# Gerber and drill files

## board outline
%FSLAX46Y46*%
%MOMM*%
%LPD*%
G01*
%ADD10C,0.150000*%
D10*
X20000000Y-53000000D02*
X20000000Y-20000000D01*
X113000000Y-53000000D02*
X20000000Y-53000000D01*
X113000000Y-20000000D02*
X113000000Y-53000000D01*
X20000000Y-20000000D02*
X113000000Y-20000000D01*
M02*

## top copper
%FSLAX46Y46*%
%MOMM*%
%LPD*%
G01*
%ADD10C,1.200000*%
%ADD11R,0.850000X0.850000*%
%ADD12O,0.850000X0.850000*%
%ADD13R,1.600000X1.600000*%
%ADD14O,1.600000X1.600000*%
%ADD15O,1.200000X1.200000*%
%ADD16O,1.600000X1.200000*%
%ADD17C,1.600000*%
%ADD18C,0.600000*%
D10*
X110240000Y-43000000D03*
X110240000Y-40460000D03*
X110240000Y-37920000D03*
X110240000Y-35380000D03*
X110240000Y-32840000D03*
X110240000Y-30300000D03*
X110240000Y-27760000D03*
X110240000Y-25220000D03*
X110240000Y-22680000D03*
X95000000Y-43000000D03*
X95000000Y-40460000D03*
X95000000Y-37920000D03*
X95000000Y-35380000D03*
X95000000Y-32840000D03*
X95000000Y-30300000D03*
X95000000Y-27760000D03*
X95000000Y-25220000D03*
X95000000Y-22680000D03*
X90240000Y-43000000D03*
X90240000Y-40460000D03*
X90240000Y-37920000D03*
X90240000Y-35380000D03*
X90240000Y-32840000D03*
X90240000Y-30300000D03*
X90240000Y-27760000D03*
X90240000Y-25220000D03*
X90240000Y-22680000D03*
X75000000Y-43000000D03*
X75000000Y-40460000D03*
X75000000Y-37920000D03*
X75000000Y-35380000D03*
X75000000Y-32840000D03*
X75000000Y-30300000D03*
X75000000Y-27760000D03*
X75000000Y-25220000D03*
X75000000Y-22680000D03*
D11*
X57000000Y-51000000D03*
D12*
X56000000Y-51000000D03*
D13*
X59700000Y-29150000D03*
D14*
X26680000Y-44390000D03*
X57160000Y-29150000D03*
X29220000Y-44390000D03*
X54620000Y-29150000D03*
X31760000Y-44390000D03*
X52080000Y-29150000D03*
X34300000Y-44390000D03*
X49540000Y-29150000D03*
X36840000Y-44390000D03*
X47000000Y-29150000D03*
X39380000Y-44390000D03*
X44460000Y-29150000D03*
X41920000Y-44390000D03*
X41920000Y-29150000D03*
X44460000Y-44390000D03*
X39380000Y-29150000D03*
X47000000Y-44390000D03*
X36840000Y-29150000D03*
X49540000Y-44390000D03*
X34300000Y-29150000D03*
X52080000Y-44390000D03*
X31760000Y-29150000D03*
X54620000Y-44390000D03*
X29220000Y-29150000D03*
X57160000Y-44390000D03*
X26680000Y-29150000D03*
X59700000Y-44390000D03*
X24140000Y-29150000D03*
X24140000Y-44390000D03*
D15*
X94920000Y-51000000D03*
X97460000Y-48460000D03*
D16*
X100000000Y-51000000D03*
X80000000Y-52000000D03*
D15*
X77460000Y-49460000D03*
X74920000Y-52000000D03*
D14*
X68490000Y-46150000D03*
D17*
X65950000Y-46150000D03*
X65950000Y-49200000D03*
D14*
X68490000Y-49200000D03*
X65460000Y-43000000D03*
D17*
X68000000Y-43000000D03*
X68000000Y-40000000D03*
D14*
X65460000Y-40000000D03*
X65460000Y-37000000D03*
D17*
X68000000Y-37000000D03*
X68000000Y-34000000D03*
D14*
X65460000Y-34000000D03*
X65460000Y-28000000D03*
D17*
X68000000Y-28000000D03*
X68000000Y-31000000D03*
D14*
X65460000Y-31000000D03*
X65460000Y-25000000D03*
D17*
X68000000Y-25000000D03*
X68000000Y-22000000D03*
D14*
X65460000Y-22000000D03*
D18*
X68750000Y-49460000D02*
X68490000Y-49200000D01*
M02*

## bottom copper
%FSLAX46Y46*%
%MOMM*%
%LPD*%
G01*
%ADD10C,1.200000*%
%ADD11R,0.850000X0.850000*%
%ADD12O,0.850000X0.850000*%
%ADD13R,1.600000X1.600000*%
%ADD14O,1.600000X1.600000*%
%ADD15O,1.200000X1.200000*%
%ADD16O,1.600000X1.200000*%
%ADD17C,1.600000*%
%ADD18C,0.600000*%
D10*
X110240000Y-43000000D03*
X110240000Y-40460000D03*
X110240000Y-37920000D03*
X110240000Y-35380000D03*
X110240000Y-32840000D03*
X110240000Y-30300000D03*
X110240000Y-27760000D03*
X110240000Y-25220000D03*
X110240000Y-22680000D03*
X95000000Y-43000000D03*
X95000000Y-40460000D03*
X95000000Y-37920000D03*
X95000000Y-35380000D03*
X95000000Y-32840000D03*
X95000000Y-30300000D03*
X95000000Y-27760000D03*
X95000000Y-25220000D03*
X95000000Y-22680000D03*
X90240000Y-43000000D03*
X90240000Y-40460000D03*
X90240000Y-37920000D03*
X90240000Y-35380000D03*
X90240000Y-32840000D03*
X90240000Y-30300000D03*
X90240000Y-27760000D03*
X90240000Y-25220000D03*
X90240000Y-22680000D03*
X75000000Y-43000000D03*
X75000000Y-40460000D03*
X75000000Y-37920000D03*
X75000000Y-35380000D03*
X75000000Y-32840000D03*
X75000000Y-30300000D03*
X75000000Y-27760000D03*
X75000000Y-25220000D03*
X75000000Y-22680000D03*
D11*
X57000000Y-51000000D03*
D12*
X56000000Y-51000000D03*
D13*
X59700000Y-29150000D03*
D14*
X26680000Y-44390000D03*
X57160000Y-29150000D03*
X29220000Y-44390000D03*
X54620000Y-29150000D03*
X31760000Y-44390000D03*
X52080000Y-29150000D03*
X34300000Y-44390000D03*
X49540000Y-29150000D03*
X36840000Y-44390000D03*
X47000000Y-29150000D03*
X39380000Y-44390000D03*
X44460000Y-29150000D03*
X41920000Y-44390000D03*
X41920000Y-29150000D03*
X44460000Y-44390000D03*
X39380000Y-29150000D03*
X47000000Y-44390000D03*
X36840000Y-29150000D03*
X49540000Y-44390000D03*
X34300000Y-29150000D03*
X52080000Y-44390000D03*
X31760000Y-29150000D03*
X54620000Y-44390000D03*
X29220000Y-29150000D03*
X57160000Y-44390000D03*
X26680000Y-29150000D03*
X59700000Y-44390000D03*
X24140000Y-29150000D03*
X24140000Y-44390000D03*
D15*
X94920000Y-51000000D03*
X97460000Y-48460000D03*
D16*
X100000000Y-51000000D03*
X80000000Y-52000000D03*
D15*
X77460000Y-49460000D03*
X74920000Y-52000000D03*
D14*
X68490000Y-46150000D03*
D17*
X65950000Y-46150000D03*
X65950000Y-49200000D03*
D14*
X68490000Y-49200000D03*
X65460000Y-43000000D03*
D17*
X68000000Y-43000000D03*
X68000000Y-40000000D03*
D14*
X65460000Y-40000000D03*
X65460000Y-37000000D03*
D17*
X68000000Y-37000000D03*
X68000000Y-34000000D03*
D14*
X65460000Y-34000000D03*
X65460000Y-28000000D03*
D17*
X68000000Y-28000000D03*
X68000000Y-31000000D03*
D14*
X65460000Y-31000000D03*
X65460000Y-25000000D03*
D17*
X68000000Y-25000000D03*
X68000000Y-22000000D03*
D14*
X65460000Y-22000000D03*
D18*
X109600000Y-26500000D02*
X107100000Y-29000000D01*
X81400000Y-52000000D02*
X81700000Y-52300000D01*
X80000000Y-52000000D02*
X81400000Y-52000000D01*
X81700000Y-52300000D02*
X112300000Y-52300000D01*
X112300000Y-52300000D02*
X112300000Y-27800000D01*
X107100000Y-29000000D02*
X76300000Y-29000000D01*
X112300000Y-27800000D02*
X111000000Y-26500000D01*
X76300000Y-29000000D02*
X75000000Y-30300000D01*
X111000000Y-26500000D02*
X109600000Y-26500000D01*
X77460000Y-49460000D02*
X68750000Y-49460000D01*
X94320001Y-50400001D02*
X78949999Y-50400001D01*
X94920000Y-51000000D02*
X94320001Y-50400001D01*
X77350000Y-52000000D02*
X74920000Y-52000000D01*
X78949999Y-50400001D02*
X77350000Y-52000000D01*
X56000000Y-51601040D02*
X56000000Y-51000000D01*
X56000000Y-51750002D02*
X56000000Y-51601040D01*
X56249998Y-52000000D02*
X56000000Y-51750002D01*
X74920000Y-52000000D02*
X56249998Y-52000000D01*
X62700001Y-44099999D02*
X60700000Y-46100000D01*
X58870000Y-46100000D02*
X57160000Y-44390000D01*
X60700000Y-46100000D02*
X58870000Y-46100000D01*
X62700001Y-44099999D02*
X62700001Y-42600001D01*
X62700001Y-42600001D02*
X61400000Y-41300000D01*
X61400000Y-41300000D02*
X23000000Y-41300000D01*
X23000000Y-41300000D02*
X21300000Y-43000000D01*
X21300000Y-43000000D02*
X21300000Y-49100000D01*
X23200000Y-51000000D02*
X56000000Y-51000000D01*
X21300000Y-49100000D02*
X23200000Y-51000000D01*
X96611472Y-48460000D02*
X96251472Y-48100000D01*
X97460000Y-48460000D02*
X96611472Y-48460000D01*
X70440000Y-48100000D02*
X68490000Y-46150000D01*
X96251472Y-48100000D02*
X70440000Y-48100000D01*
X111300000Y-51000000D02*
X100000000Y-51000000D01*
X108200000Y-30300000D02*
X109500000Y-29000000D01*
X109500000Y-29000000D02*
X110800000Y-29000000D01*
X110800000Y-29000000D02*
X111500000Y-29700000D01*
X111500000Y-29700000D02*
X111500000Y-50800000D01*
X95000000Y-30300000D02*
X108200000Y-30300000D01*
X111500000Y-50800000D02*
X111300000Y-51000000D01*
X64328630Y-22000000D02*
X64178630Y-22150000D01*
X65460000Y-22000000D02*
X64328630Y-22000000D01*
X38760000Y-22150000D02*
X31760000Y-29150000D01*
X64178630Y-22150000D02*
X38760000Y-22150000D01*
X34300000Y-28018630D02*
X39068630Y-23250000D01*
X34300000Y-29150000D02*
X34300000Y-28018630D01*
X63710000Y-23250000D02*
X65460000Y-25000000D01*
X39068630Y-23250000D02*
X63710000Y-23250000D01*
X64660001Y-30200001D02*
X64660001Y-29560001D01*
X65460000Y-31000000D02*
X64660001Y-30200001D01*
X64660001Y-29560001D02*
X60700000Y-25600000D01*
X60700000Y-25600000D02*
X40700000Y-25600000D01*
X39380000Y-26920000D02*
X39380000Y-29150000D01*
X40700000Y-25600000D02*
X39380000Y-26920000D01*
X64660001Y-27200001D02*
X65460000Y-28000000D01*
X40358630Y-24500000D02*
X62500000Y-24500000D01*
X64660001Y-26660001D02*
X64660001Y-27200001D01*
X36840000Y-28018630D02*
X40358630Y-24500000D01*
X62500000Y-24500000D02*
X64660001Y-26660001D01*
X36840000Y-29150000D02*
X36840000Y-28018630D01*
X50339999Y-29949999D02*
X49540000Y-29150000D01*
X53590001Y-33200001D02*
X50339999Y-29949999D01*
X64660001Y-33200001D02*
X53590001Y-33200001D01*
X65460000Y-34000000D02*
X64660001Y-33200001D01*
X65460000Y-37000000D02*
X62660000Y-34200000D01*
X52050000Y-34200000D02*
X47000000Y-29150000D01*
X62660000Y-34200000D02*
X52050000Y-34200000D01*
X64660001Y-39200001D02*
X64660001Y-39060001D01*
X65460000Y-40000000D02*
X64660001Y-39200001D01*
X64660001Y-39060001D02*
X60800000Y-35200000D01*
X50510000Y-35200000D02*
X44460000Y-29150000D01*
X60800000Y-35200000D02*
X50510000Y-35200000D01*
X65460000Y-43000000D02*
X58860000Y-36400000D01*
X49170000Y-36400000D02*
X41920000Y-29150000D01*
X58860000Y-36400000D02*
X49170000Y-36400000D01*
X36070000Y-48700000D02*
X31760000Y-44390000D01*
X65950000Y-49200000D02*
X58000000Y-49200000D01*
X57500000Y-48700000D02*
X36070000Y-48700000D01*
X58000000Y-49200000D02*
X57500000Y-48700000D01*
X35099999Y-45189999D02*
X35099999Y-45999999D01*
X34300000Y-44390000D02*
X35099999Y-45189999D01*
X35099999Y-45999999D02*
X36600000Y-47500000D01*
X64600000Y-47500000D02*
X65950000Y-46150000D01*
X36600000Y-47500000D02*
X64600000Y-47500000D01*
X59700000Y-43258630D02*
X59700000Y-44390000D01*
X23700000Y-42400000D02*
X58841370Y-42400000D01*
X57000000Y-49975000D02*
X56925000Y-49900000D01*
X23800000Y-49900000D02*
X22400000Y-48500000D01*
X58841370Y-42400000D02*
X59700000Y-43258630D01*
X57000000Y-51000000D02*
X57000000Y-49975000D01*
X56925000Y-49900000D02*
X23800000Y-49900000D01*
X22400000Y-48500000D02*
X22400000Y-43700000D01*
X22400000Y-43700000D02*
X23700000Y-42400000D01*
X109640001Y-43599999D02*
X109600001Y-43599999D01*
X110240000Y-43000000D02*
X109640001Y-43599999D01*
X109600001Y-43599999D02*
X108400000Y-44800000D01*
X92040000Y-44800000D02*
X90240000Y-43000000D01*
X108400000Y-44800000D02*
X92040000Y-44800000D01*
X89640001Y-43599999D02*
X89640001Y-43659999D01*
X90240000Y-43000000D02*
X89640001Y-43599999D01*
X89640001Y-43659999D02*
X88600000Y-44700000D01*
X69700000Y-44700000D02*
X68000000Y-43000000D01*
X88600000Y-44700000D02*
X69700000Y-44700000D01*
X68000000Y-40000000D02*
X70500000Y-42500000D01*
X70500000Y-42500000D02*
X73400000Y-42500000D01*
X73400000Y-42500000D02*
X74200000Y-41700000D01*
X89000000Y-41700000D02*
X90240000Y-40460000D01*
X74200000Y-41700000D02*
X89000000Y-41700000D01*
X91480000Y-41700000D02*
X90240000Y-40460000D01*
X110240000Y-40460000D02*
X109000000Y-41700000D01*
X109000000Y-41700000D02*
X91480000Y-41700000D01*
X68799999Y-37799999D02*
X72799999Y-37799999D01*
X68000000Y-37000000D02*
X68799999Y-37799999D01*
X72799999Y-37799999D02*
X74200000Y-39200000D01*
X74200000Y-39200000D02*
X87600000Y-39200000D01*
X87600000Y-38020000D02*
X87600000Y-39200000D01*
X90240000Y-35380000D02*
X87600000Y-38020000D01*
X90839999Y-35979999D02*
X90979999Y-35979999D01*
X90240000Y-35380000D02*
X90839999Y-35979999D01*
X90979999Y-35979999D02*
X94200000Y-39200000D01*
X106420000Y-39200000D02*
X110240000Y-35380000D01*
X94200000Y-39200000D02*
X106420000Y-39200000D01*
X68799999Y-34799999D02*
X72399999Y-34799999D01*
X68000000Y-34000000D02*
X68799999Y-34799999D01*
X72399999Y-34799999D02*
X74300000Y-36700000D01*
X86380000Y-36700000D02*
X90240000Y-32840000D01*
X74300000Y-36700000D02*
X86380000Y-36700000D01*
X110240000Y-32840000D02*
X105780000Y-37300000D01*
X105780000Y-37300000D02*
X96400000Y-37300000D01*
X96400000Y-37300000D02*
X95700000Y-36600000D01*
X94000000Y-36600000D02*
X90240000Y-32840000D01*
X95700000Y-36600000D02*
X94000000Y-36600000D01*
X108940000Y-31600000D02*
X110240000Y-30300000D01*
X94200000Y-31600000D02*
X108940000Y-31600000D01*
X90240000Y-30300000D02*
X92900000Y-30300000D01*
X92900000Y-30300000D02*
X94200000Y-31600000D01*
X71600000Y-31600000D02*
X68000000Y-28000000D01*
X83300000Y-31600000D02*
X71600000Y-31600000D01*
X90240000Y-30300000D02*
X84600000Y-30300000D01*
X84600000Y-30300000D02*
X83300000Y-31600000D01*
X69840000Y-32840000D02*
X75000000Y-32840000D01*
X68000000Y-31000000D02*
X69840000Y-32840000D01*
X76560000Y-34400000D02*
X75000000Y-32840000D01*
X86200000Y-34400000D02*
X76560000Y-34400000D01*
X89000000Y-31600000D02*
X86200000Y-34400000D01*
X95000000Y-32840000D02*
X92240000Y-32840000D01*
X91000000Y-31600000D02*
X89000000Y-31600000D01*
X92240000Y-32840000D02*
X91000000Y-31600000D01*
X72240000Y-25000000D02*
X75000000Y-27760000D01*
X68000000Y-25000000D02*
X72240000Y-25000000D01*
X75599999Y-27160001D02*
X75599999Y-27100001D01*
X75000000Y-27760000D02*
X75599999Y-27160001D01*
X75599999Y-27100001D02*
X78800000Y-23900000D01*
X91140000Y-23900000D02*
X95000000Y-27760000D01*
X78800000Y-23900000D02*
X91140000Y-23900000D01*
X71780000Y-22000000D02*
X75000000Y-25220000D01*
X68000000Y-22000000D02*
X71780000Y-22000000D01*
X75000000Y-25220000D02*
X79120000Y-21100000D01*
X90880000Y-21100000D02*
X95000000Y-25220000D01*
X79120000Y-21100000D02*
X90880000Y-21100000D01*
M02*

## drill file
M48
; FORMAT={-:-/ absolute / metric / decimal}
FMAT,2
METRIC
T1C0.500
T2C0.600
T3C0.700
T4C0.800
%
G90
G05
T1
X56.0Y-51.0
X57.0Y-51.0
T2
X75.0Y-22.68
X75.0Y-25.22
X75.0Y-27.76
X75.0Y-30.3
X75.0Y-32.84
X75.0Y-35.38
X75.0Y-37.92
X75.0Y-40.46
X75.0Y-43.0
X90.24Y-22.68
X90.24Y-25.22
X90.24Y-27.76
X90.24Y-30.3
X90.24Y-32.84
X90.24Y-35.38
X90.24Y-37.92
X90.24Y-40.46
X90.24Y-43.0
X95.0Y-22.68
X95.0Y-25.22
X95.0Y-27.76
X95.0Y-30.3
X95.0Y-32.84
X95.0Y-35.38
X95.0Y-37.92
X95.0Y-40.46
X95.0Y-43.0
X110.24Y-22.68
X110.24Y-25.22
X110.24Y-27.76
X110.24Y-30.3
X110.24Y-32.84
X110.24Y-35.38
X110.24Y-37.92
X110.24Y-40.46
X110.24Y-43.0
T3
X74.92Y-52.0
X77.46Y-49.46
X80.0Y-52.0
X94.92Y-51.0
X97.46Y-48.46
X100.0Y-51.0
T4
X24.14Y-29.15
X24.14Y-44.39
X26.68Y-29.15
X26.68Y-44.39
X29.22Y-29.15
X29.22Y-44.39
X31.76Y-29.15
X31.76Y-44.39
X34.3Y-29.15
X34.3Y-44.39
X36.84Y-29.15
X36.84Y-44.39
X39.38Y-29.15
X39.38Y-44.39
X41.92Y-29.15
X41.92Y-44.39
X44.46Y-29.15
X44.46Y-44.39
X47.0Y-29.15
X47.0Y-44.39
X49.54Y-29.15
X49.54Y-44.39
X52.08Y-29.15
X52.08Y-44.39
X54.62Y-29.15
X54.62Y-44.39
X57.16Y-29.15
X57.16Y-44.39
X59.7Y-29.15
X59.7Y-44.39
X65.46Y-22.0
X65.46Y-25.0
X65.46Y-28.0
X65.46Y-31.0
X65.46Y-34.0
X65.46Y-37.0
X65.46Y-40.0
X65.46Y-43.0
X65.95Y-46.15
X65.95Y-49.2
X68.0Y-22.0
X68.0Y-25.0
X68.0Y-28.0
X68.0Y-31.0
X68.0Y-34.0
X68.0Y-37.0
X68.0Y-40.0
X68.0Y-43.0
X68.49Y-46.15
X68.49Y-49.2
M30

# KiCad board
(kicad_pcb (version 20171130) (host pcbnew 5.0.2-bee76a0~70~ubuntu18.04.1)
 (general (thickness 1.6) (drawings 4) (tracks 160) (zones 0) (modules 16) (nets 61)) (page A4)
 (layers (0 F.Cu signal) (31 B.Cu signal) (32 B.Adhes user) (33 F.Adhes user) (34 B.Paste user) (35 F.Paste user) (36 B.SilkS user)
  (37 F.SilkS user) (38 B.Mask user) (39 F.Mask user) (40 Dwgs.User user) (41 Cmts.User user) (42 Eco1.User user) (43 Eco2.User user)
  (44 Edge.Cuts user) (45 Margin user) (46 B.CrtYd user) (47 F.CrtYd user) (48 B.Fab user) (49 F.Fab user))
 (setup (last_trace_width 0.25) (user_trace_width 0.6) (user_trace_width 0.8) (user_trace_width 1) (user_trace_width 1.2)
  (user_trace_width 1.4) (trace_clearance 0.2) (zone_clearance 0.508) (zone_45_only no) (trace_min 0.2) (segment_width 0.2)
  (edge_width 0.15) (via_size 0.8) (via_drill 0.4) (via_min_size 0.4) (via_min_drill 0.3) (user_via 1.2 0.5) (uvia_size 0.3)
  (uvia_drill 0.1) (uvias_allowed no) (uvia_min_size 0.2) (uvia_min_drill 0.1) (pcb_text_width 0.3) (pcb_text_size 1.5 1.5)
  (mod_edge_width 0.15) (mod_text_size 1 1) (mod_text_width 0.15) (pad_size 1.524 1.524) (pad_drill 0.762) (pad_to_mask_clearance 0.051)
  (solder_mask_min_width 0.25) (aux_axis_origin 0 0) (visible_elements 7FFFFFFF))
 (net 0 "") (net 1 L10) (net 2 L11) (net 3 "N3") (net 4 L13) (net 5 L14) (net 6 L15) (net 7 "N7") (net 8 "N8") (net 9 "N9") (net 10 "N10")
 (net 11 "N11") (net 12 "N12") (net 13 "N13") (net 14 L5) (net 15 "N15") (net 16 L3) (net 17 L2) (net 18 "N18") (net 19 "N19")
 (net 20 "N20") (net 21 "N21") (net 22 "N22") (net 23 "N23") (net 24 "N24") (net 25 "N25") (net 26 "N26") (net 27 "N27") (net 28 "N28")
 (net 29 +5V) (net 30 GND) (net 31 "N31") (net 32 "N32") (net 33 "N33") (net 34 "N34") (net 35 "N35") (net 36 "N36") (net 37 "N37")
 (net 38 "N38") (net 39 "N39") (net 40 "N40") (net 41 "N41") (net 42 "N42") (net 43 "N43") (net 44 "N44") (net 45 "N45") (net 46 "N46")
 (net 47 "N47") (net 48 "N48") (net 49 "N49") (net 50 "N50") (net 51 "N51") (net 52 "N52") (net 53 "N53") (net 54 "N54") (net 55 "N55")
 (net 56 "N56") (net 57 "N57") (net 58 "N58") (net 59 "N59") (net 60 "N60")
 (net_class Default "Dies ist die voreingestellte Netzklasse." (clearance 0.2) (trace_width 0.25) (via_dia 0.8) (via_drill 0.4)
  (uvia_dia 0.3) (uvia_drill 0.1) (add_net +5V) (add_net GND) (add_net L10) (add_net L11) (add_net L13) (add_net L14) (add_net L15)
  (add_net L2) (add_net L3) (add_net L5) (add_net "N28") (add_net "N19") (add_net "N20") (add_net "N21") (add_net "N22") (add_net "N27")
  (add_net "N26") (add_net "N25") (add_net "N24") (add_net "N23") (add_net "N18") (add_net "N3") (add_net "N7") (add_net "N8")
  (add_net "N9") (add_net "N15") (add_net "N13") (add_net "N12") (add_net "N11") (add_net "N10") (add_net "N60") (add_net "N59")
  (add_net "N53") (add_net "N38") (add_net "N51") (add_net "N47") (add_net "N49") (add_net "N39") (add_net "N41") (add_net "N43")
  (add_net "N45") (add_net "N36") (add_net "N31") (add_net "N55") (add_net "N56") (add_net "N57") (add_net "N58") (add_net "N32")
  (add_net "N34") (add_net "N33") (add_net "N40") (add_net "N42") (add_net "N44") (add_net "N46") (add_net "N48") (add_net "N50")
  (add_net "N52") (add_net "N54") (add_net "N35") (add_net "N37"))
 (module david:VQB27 (layer F.Cu) (at 95 43)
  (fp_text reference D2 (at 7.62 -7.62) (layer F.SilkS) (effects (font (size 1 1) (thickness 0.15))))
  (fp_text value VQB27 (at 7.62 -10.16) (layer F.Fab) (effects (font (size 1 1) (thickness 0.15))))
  (pad 10 thru_hole circle (at 15.24 0) (size 1.2 1.2) (drill 0.6) (layers *.Cu *.Mask) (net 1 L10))
  (pad 11 thru_hole circle (at 15.24 -2.54) (size 1.2 1.2) (drill 0.6) (layers *.Cu *.Mask) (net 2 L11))
  (pad 12 thru_hole circle (at 15.24 -5.08) (size 1.2 1.2) (drill 0.6) (layers *.Cu *.Mask) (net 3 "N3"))
  (pad 13 thru_hole circle (at 15.24 -7.62) (size 1.2 1.2) (drill 0.6) (layers *.Cu *.Mask) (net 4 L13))
  (pad 14 thru_hole circle (at 15.24 -10.16) (size 1.2 1.2) (drill 0.6) (layers *.Cu *.Mask) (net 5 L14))
  (pad 15 thru_hole circle (at 15.24 -12.7) (size 1.2 1.2) (drill 0.6) (layers *.Cu *.Mask) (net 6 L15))
  (pad 16 thru_hole circle (at 15.24 -15.24) (size 1.2 1.2) (drill 0.6) (layers *.Cu *.Mask) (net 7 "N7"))
  (pad 17 thru_hole circle (at 15.24 -17.78) (size 1.2 1.2) (drill 0.6) (layers *.Cu *.Mask) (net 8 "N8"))
  (pad 18 thru_hole circle (at 15.24 -20.32) (size 1.2 1.2) (drill 0.6) (layers *.Cu *.Mask) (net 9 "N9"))
  (pad 9 thru_hole circle (at 0 0) (size 1.2 1.2) (drill 0.6) (layers *.Cu *.Mask) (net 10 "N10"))
  (pad 8 thru_hole circle (at 0 -2.54) (size 1.2 1.2) (drill 0.6) (layers *.Cu *.Mask) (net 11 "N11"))
  (pad 7 thru_hole circle (at 0 -5.08) (size 1.2 1.2) (drill 0.6) (layers *.Cu *.Mask) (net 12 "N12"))
  (pad 6 thru_hole circle (at 0 -7.62) (size 1.2 1.2) (drill 0.6) (layers *.Cu *.Mask) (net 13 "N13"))
  (pad 5 thru_hole circle (at 0 -10.16) (size 1.2 1.2) (drill 0.6) (layers *.Cu *.Mask) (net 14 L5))
  (pad 4 thru_hole circle (at 0 -12.7) (size 1.2 1.2) (drill 0.6) (layers *.Cu *.Mask) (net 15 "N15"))
  (pad 3 thru_hole circle (at 0 -15.24) (size 1.2 1.2) (drill 0.6) (layers *.Cu *.Mask) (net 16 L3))
  (pad 2 thru_hole circle (at 0 -17.78) (size 1.2 1.2) (drill 0.6) (layers *.Cu *.Mask) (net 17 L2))
  (pad 1 thru_hole circle (at 0 -20.32) (size 1.2 1.2) (drill 0.6) (layers *.Cu *.Mask) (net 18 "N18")))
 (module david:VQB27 (layer F.Cu) (at 75 43)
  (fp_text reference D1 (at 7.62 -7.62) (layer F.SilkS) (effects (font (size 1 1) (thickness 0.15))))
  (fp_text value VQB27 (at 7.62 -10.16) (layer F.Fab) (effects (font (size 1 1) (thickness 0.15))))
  (pad 10 thru_hole circle (at 15.24 0) (size 1.2 1.2) (drill 0.6) (layers *.Cu *.Mask) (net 1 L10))
  (pad 11 thru_hole circle (at 15.24 -2.54) (size 1.2 1.2) (drill 0.6) (layers *.Cu *.Mask) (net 2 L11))
  (pad 12 thru_hole circle (at 15.24 -5.08) (size 1.2 1.2) (drill 0.6) (layers *.Cu *.Mask) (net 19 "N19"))
  (pad 13 thru_hole circle (at 15.24 -7.62) (size 1.2 1.2) (drill 0.6) (layers *.Cu *.Mask) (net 4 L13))
  (pad 14 thru_hole circle (at 15.24 -10.16) (size 1.2 1.2) (drill 0.6) (layers *.Cu *.Mask) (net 5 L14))
  (pad 15 thru_hole circle (at 15.24 -12.7) (size 1.2 1.2) (drill 0.6) (layers *.Cu *.Mask) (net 6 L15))
  (pad 16 thru_hole circle (at 15.24 -15.24) (size 1.2 1.2) (drill 0.6) (layers *.Cu *.Mask) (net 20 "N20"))
  (pad 17 thru_hole circle (at 15.24 -17.78) (size 1.2 1.2) (drill 0.6) (layers *.Cu *.Mask) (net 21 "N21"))
  (pad 18 thru_hole circle (at 15.24 -20.32) (size 1.2 1.2) (drill 0.6) (layers *.Cu *.Mask) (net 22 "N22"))
  (pad 9 thru_hole circle (at 0 0) (size 1.2 1.2) (drill 0.6) (layers *.Cu *.Mask) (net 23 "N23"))
  (pad 8 thru_hole circle (at 0 -2.54) (size 1.2 1.2) (drill 0.6) (layers *.Cu *.Mask) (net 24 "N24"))
  (pad 7 thru_hole circle (at 0 -5.08) (size 1.2 1.2) (drill 0.6) (layers *.Cu *.Mask) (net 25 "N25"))
  (pad 6 thru_hole circle (at 0 -7.62) (size 1.2 1.2) (drill 0.6) (layers *.Cu *.Mask) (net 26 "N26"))
  (pad 5 thru_hole circle (at 0 -10.16) (size 1.2 1.2) (drill 0.6) (layers *.Cu *.Mask) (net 14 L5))
  (pad 4 thru_hole circle (at 0 -12.7) (size 1.2 1.2) (drill 0.6) (layers *.Cu *.Mask) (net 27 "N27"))
  (pad 3 thru_hole circle (at 0 -15.24) (size 1.2 1.2) (drill 0.6) (layers *.Cu *.Mask) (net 16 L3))
  (pad 2 thru_hole circle (at 0 -17.78) (size 1.2 1.2) (drill 0.6) (layers *.Cu *.Mask) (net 17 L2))
  (pad 1 thru_hole circle (at 0 -20.32) (size 1.2 1.2) (drill 0.6) (layers *.Cu *.Mask) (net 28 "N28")))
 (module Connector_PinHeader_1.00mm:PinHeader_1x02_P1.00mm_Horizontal (layer F.Cu) (at 57 51 270)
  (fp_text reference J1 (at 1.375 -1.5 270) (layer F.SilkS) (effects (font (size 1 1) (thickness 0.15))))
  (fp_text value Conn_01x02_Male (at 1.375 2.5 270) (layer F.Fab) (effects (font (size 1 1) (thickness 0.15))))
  (pad 1 thru_hole rect (at 0 0 270) (size 0.85 0.85) (drill 0.5) (layers *.Cu *.Mask) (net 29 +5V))
  (pad 2 thru_hole oval (at 0 1 270) (size 0.85 0.85) (drill 0.5) (layers *.Cu *.Mask) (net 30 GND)))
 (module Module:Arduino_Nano (layer F.Cu) (at 59.7 29.15 270)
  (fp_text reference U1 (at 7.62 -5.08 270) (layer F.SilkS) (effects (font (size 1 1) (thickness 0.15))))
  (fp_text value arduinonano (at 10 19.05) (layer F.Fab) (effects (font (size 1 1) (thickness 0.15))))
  (pad 1 thru_hole rect (at 0 0 270) (size 1.6 1.6) (drill 0.8) (layers *.Cu *.Mask) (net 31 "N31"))
  (pad 17 thru_hole oval (at 15.24 33.02 270) (size 1.6 1.6) (drill 0.8) (layers *.Cu *.Mask) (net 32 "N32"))
  (pad 2 thru_hole oval (at 0 2.54 270) (size 1.6 1.6) (drill 0.8) (layers *.Cu *.Mask) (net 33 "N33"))
  (pad 18 thru_hole oval (at 15.24 30.48 270) (size 1.6 1.6) (drill 0.8) (layers *.Cu *.Mask) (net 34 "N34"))
  (pad 3 thru_hole oval (at 0 5.08 270) (size 1.6 1.6) (drill 0.8) (layers *.Cu *.Mask) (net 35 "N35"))
  (pad 19 thru_hole oval (at 15.24 27.94 270) (size 1.6 1.6) (drill 0.8) (layers *.Cu *.Mask) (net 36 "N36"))
  (pad 4 thru_hole oval (at 0 7.62 270) (size 1.6 1.6) (drill 0.8) (layers *.Cu *.Mask) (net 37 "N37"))
  (pad 20 thru_hole oval (at 15.24 25.4 270) (size 1.6 1.6) (drill 0.8) (layers *.Cu *.Mask) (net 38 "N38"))
  (pad 5 thru_hole oval (at 0 10.16 270) (size 1.6 1.6) (drill 0.8) (layers *.Cu *.Mask) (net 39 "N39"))
  (pad 21 thru_hole oval (at 15.24 22.86 270) (size 1.6 1.6) (drill 0.8) (layers *.Cu *.Mask) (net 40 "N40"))
  (pad 6 thru_hole oval (at 0 12.7 270) (size 1.6 1.6) (drill 0.8) (layers *.Cu *.Mask) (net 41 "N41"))
  (pad 22 thru_hole oval (at 15.24 20.32 270) (size 1.6 1.6) (drill 0.8) (layers *.Cu *.Mask) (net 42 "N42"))
  (pad 7 thru_hole oval (at 0 15.24 270) (size 1.6 1.6) (drill 0.8) (layers *.Cu *.Mask) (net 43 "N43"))
  (pad 23 thru_hole oval (at 15.24 17.78 270) (size 1.6 1.6) (drill 0.8) (layers *.Cu *.Mask) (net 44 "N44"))
  (pad 8 thru_hole oval (at 0 17.78 270) (size 1.6 1.6) (drill 0.8) (layers *.Cu *.Mask) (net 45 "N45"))
  (pad 24 thru_hole oval (at 15.24 15.24 270) (size 1.6 1.6) (drill 0.8) (layers *.Cu *.Mask) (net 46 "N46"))
  (pad 9 thru_hole oval (at 0 20.32 270) (size 1.6 1.6) (drill 0.8) (layers *.Cu *.Mask) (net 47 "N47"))
  (pad 25 thru_hole oval (at 15.24 12.7 270) (size 1.6 1.6) (drill 0.8) (layers *.Cu *.Mask) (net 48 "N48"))
  (pad 10 thru_hole oval (at 0 22.86 270) (size 1.6 1.6) (drill 0.8) (layers *.Cu *.Mask) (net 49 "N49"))
  (pad 26 thru_hole oval (at 15.24 10.16 270) (size 1.6 1.6) (drill 0.8) (layers *.Cu *.Mask) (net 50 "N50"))
  (pad 11 thru_hole oval (at 0 25.4 270) (size 1.6 1.6) (drill 0.8) (layers *.Cu *.Mask) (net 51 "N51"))
  (pad 27 thru_hole oval (at 15.24 7.62 270) (size 1.6 1.6) (drill 0.8) (layers *.Cu *.Mask) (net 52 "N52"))
  (pad 12 thru_hole oval (at 0 27.94 270) (size 1.6 1.6) (drill 0.8) (layers *.Cu *.Mask) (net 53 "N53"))
  (pad 28 thru_hole oval (at 15.24 5.08 270) (size 1.6 1.6) (drill 0.8) (layers *.Cu *.Mask) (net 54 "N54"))
  (pad 13 thru_hole oval (at 0 30.48 270) (size 1.6 1.6) (drill 0.8) (layers *.Cu *.Mask) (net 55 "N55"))
  (pad 29 thru_hole oval (at 15.24 2.54 270) (size 1.6 1.6) (drill 0.8) (layers *.Cu *.Mask) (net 30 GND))
  (pad 14 thru_hole oval (at 0 33.02 270) (size 1.6 1.6) (drill 0.8) (layers *.Cu *.Mask) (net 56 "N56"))
  (pad 30 thru_hole oval (at 15.24 0 270) (size 1.6 1.6) (drill 0.8) (layers *.Cu *.Mask) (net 29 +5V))
  (pad 15 thru_hole oval (at 0 35.56 270) (size 1.6 1.6) (drill 0.8) (layers *.Cu *.Mask) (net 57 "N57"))
  (pad 16 thru_hole oval (at 15.24 35.56 270) (size 1.6 1.6) (drill 0.8) (layers *.Cu *.Mask) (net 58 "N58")))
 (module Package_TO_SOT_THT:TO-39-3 (layer F.Cu) (at 100 51 180)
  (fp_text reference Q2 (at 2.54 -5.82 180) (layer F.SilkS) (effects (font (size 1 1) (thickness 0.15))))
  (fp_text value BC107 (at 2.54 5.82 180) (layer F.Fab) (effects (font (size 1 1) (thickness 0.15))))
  (pad 3 thru_hole oval (at 5.08 0 180) (size 1.2 1.2) (drill 0.7) (layers *.Cu *.Mask) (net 30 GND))
  (pad 2 thru_hole oval (at 2.54 2.54 180) (size 1.2 1.2) (drill 0.7) (layers *.Cu *.Mask) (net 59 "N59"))
  (pad 1 thru_hole oval (at 0 0 180) (size 1.6 1.2) (drill 0.7) (layers *.Cu *.Mask) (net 15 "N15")))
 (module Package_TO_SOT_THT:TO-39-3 (layer F.Cu) (at 80 52 180)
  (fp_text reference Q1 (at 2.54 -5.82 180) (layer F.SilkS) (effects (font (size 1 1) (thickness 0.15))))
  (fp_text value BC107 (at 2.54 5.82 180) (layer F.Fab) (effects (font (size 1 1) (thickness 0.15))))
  (pad 1 thru_hole oval (at 0 0 180) (size 1.6 1.2) (drill 0.7) (layers *.Cu *.Mask) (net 27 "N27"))
  (pad 2 thru_hole oval (at 2.54 2.54 180) (size 1.2 1.2) (drill 0.7) (layers *.Cu *.Mask) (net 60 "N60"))
  (pad 3 thru_hole oval (at 5.08 0 180) (size 1.2 1.2) (drill 0.7) (layers *.Cu *.Mask) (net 30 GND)))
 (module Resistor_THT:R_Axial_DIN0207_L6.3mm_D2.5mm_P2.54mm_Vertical (layer F.Cu) (at 65.95 46.15)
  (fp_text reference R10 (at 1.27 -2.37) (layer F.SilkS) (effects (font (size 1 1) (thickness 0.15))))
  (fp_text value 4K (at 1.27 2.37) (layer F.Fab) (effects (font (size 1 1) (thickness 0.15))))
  (pad 2 thru_hole oval (at 2.54 0) (size 1.6 1.6) (drill 0.8) (layers *.Cu *.Mask) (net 59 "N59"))
  (pad 1 thru_hole circle (at 0 0) (size 1.6 1.6) (drill 0.8) (layers *.Cu *.Mask) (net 38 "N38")))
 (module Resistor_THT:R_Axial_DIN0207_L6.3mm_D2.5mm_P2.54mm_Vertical (layer F.Cu) (at 65.95 49.2)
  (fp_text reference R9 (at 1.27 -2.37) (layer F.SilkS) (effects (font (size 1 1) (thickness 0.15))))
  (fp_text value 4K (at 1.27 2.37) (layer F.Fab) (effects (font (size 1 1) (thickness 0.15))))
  (pad 1 thru_hole circle (at 0 0) (size 1.6 1.6) (drill 0.8) (layers *.Cu *.Mask) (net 36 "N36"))
  (pad 2 thru_hole oval (at 2.54 0) (size 1.6 1.6) (drill 0.8) (layers *.Cu *.Mask) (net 60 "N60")))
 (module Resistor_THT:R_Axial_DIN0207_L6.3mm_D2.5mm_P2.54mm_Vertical (layer F.Cu) (at 68 43 180)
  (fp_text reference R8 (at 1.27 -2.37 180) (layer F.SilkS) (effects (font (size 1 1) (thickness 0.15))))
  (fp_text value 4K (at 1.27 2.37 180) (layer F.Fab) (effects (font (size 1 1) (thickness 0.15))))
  (pad 2 thru_hole oval (at 2.54 0 180) (size 1.6 1.6) (drill 0.8) (layers *.Cu *.Mask) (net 45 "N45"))
  (pad 1 thru_hole circle (at 0 0 180) (size 1.6 1.6) (drill 0.8) (layers *.Cu *.Mask) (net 1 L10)))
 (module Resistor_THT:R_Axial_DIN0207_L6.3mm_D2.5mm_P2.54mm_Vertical (layer F.Cu) (at 68 40 180)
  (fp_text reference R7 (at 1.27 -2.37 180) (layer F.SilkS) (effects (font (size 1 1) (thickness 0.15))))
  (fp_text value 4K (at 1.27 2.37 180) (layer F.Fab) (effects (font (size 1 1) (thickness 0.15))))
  (pad 1 thru_hole circle (at 0 0 180) (size 1.6 1.6) (drill 0.8) (layers *.Cu *.Mask) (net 2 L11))
  (pad 2 thru_hole oval (at 2.54 0 180) (size 1.6 1.6) (drill 0.8) (layers *.Cu *.Mask) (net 43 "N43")))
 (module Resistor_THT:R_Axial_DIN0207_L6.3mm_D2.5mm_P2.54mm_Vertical (layer F.Cu) (at 68 37 180)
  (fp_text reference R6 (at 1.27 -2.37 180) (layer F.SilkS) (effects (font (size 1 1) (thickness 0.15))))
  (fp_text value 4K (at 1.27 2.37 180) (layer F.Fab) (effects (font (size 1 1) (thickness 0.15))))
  (pad 2 thru_hole oval (at 2.54 0 180) (size 1.6 1.6) (drill 0.8) (layers *.Cu *.Mask) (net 41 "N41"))
  (pad 1 thru_hole circle (at 0 0 180) (size 1.6 1.6) (drill 0.8) (layers *.Cu *.Mask) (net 4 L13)))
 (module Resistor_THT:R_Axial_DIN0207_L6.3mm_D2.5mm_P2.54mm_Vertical (layer F.Cu) (at 68 34 180)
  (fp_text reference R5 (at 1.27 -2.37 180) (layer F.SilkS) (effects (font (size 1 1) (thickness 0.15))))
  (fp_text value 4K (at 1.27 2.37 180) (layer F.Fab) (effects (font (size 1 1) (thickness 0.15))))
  (pad 1 thru_hole circle (at 0 0 180) (size 1.6 1.6) (drill 0.8) (layers *.Cu *.Mask) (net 5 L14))
  (pad 2 thru_hole oval (at 2.54 0 180) (size 1.6 1.6) (drill 0.8) (layers *.Cu *.Mask) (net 39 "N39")))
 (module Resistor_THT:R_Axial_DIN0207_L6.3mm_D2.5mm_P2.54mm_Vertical (layer F.Cu) (at 68 28 180)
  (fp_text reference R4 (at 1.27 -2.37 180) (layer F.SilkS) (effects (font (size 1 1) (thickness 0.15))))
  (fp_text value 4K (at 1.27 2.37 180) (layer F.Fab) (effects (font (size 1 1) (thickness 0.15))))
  (pad 2 thru_hole oval (at 2.54 0 180) (size 1.6 1.6) (drill 0.8) (layers *.Cu *.Mask) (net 49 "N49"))
  (pad 1 thru_hole circle (at 0 0 180) (size 1.6 1.6) (drill 0.8) (layers *.Cu *.Mask) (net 6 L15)))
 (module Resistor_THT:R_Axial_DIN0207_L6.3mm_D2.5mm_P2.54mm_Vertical (layer F.Cu) (at 68 31 180)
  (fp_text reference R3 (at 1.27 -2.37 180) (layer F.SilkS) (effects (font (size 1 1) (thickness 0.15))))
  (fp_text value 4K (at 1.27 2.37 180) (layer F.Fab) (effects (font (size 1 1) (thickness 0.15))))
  (pad 1 thru_hole circle (at 0 0 180) (size 1.6 1.6) (drill 0.8) (layers *.Cu *.Mask) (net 14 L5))
  (pad 2 thru_hole oval (at 2.54 0 180) (size 1.6 1.6) (drill 0.8) (layers *.Cu *.Mask) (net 47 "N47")))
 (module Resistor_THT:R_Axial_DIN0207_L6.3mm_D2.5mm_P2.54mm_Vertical (layer F.Cu) (at 68 25 180)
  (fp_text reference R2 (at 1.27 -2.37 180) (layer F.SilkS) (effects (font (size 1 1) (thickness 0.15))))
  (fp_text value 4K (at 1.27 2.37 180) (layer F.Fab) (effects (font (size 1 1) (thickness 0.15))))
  (pad 2 thru_hole oval (at 2.54 0 180) (size 1.6 1.6) (drill 0.8) (layers *.Cu *.Mask) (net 51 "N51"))
  (pad 1 thru_hole circle (at 0 0 180) (size 1.6 1.6) (drill 0.8) (layers *.Cu *.Mask) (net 16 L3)))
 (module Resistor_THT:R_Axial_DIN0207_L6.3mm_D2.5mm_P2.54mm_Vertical (layer F.Cu) (at 68 22 180)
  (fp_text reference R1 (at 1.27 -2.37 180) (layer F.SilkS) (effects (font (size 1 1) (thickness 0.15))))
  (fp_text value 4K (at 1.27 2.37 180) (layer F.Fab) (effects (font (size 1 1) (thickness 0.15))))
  (pad 1 thru_hole circle (at 0 0 180) (size 1.6 1.6) (drill 0.8) (layers *.Cu *.Mask) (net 17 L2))
  (pad 2 thru_hole oval (at 2.54 0 180) (size 1.6 1.6) (drill 0.8) (layers *.Cu *.Mask) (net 53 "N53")))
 (gr_line (start 20 53) (end 20 20) (layer Edge.Cuts) (width 0.15))
 (gr_line (start 113 53) (end 20 53) (layer Edge.Cuts) (width 0.15))
 (gr_line (start 113 20) (end 113 53) (layer Edge.Cuts) (width 0.15))
 (gr_line (start 20 20) (end 113 20) (layer Edge.Cuts) (width 0.15))
 (segment (start 109.6 26.5) (end 107.1 29) (width 0.6) (layer B.Cu) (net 27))
 (segment (start 81.4 52) (end 81.7 52.3) (width 0.6) (layer B.Cu) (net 27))
 (segment (start 80 52) (end 81.4 52) (width 0.6) (layer B.Cu) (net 27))
 (segment (start 81.7 52.3) (end 112.3 52.3) (width 0.6) (layer B.Cu) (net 27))
 (segment (start 112.3 52.3) (end 112.3 27.8) (width 0.6) (layer B.Cu) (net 27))
 (segment (start 107.1 29) (end 76.3 29) (width 0.6) (layer B.Cu) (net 27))
 (segment (start 112.3 27.8) (end 111 26.5) (width 0.6) (layer B.Cu) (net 27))
 (segment (start 76.3 29) (end 75 30.3) (width 0.6) (layer B.Cu) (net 27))
 (segment (start 111 26.5) (end 109.6 26.5) (width 0.6) (layer B.Cu) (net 27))
 (segment (start 68.75 49.46) (end 68.49 49.2) (width 0.6) (layer F.Cu) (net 60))
 (segment (start 77.46 49.46) (end 68.75 49.46) (width 0.6) (layer B.Cu) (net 60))
 (segment (start 94.320001 50.400001) (end 78.949999 50.400001) (width 0.6) (layer B.Cu) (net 30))
 (segment (start 94.92 51) (end 94.320001 50.400001) (width 0.6) (layer B.Cu) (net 30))
 (segment (start 77.35 52) (end 74.92 52) (width 0.6) (layer B.Cu) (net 30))
 (segment (start 78.949999 50.400001) (end 77.35 52) (width 0.6) (layer B.Cu) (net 30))
 (segment (start 56 51.60104) (end 56 51) (width 0.6) (layer B.Cu) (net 30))
 (segment (start 56 51.750002) (end 56 51.60104) (width 0.6) (layer B.Cu) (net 30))
 (segment (start 56.249998 52) (end 56 51.750002) (width 0.6) (layer B.Cu) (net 30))
 (segment (start 74.92 52) (end 56.249998 52) (width 0.6) (layer B.Cu) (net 30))
 (segment (start 62.700001 44.099999) (end 60.7 46.1) (width 0.6) (layer B.Cu) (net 30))
 (segment (start 58.87 46.1) (end 57.16 44.39) (width 0.6) (layer B.Cu) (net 30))
 (segment (start 60.7 46.1) (end 58.87 46.1) (width 0.6) (layer B.Cu) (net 30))
 (segment (start 62.700001 44.099999) (end 62.700001 42.600001) (width 0.6) (layer B.Cu) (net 30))
 (segment (start 62.700001 42.600001) (end 61.4 41.3) (width 0.6) (layer B.Cu) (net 30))
 (segment (start 61.4 41.3) (end 23 41.3) (width 0.6) (layer B.Cu) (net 30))
 (segment (start 23 41.3) (end 21.3 43) (width 0.6) (layer B.Cu) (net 30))
 (segment (start 21.3 43) (end 21.3 49.1) (width 0.6) (layer B.Cu) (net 30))
 (segment (start 23.2 51) (end 56 51) (width 0.6) (layer B.Cu) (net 30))
 (segment (start 21.3 49.1) (end 23.2 51) (width 0.6) (layer B.Cu) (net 30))
 (segment (start 96.611472 48.46) (end 96.251472 48.1) (width 0.6) (layer B.Cu) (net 59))
 (segment (start 97.46 48.46) (end 96.611472 48.46) (width 0.6) (layer B.Cu) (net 59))
 (segment (start 70.44 48.1) (end 68.49 46.15) (width 0.6) (layer B.Cu) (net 59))
 (segment (start 96.251472 48.1) (end 70.44 48.1) (width 0.6) (layer B.Cu) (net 59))
 (segment (start 111.3 51) (end 100 51) (width 0.6) (layer B.Cu) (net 15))
 (segment (start 108.2 30.3) (end 109.5 29) (width 0.6) (layer B.Cu) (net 15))
 (segment (start 109.5 29) (end 110.8 29) (width 0.6) (layer B.Cu) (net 15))
 (segment (start 110.8 29) (end 111.5 29.7) (width 0.6) (layer B.Cu) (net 15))
 (segment (start 111.5 29.7) (end 111.5 50.8) (width 0.6) (layer B.Cu) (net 15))
 (segment (start 95 30.3) (end 108.2 30.3) (width 0.6) (layer B.Cu) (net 15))
 (segment (start 111.5 50.8) (end 111.3 51) (width 0.6) (layer B.Cu) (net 15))
 (segment (start 64.32863 22) (end 64.17863 22.15) (width 0.6) (layer B.Cu) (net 53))
 (segment (start 65.46 22) (end 64.32863 22) (width 0.6) (layer B.Cu) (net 53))
 (segment (start 38.76 22.15) (end 31.76 29.15) (width 0.6) (layer B.Cu) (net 53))
 (segment (start 64.17863 22.15) (end 38.76 22.15) (width 0.6) (layer B.Cu) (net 53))
 (segment (start 34.3 28.01863) (end 39.06863 23.25) (width 0.6) (layer B.Cu) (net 51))
 (segment (start 34.3 29.15) (end 34.3 28.01863) (width 0.6) (layer B.Cu) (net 51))
 (segment (start 63.71 23.25) (end 65.46 25) (width 0.6) (layer B.Cu) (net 51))
 (segment (start 39.06863 23.25) (end 63.71 23.25) (width 0.6) (layer B.Cu) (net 51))
 (segment (start 64.660001 30.200001) (end 64.660001 29.560001) (width 0.6) (layer B.Cu) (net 47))
 (segment (start 65.46 31) (end 64.660001 30.200001) (width 0.6) (layer B.Cu) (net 47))
 (segment (start 64.660001 29.560001) (end 60.7 25.6) (width 0.6) (layer B.Cu) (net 47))
 (segment (start 60.7 25.6) (end 40.7 25.6) (width 0.6) (layer B.Cu) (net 47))
 (segment (start 39.38 26.92) (end 39.38 29.15) (width 0.6) (layer B.Cu) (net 47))
 (segment (start 40.7 25.6) (end 39.38 26.92) (width 0.6) (layer B.Cu) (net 47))
 (segment (start 64.660001 27.200001) (end 65.46 28) (width 0.6) (layer B.Cu) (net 49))
 (segment (start 40.35863 24.5) (end 62.5 24.5) (width 0.6) (layer B.Cu) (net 49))
 (segment (start 64.660001 26.660001) (end 64.660001 27.200001) (width 0.6) (layer B.Cu) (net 49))
 (segment (start 36.84 28.01863) (end 40.35863 24.5) (width 0.6) (layer B.Cu) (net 49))
 (segment (start 62.5 24.5) (end 64.660001 26.660001) (width 0.6) (layer B.Cu) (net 49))
 (segment (start 36.84 29.15) (end 36.84 28.01863) (width 0.6) (layer B.Cu) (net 49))
 (segment (start 50.339999 29.949999) (end 49.54 29.15) (width 0.6) (layer B.Cu) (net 39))
 (segment (start 53.590001 33.200001) (end 50.339999 29.949999) (width 0.6) (layer B.Cu) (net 39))
 (segment (start 64.660001 33.200001) (end 53.590001 33.200001) (width 0.6) (layer B.Cu) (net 39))
 (segment (start 65.46 34) (end 64.660001 33.200001) (width 0.6) (layer B.Cu) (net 39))
 (segment (start 65.46 37) (end 62.66 34.2) (width 0.6) (layer B.Cu) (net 41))
 (segment (start 52.05 34.2) (end 47 29.15) (width 0.6) (layer B.Cu) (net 41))
 (segment (start 62.66 34.2) (end 52.05 34.2) (width 0.6) (layer B.Cu) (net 41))
 (segment (start 64.660001 39.200001) (end 64.660001 39.060001) (width 0.6) (layer B.Cu) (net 43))
 (segment (start 65.46 40) (end 64.660001 39.200001) (width 0.6) (layer B.Cu) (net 43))
 (segment (start 64.660001 39.060001) (end 60.8 35.2) (width 0.6) (layer B.Cu) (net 43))
 (segment (start 50.51 35.2) (end 44.46 29.15) (width 0.6) (layer B.Cu) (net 43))
 (segment (start 60.8 35.2) (end 50.51 35.2) (width 0.6) (layer B.Cu) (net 43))
 (segment (start 65.46 43) (end 58.86 36.4) (width 0.6) (layer B.Cu) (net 45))
 (segment (start 49.17 36.4) (end 41.92 29.15) (width 0.6) (layer B.Cu) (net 45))
 (segment (start 58.86 36.4) (end 49.17 36.4) (width 0.6) (layer B.Cu) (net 45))
 (segment (start 36.07 48.7) (end 31.76 44.39) (width 0.6) (layer B.Cu) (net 36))
 (segment (start 65.95 49.2) (end 58 49.2) (width 0.6) (layer B.Cu) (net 36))
 (segment (start 57.5 48.7) (end 36.07 48.7) (width 0.6) (layer B.Cu) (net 36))
 (segment (start 58 49.2) (end 57.5 48.7) (width 0.6) (layer B.Cu) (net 36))
 (segment (start 35.099999 45.189999) (end 35.099999 45.999999) (width 0.6) (layer B.Cu) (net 38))
 (segment (start 34.3 44.39) (end 35.099999 45.189999) (width 0.6) (layer B.Cu) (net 38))
 (segment (start 35.099999 45.999999) (end 36.6 47.5) (width 0.6) (layer B.Cu) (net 38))
 (segment (start 64.6 47.5) (end 65.95 46.15) (width 0.6) (layer B.Cu) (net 38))
 (segment (start 36.6 47.5) (end 64.6 47.5) (width 0.6) (layer B.Cu) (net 38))
 (segment (start 59.7 43.25863) (end 59.7 44.39) (width 0.6) (layer B.Cu) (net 29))
 (segment (start 23.7 42.4) (end 58.84137 42.4) (width 0.6) (layer B.Cu) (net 29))
 (segment (start 57 49.975) (end 56.925 49.9) (width 0.6) (layer B.Cu) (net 29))
 (segment (start 23.8 49.9) (end 22.4 48.5) (width 0.6) (layer B.Cu) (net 29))
 (segment (start 58.84137 42.4) (end 59.7 43.25863) (width 0.6) (layer B.Cu) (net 29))
 (segment (start 57 51) (end 57 49.975) (width 0.6) (layer B.Cu) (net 29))
 (segment (start 56.925 49.9) (end 23.8 49.9) (width 0.6) (layer B.Cu) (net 29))
 (segment (start 22.4 48.5) (end 22.4 43.7) (width 0.6) (layer B.Cu) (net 29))
 (segment (start 22.4 43.7) (end 23.7 42.4) (width 0.6) (layer B.Cu) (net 29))
 (segment (start 109.640001 43.599999) (end 109.600001 43.599999) (width 0.6) (layer B.Cu) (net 1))
 (segment (start 110.24 43) (end 109.640001 43.599999) (width 0.6) (layer B.Cu) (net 1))
 (segment (start 109.600001 43.599999) (end 108.4 44.8) (width 0.6) (layer B.Cu) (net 1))
 (segment (start 92.04 44.8) (end 90.24 43) (width 0.6) (layer B.Cu) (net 1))
 (segment (start 108.4 44.8) (end 92.04 44.8) (width 0.6) (layer B.Cu) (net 1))
 (segment (start 89.640001 43.599999) (end 89.640001 43.659999) (width 0.6) (layer B.Cu) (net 1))
 (segment (start 90.24 43) (end 89.640001 43.599999) (width 0.6) (layer B.Cu) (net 1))
 (segment (start 89.640001 43.659999) (end 88.6 44.7) (width 0.6) (layer B.Cu) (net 1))
 (segment (start 69.7 44.7) (end 68 43) (width 0.6) (layer B.Cu) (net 1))
 (segment (start 88.6 44.7) (end 69.7 44.7) (width 0.6) (layer B.Cu) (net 1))
 (segment (start 68 40) (end 70.5 42.5) (width 0.6) (layer B.Cu) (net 2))
 (segment (start 70.5 42.5) (end 73.4 42.5) (width 0.6) (layer B.Cu) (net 2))
 (segment (start 73.4 42.5) (end 74.2 41.7) (width 0.6) (layer B.Cu) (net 2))
 (segment (start 89 41.7) (end 90.24 40.46) (width 0.6) (layer B.Cu) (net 2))
 (segment (start 74.2 41.7) (end 89 41.7) (width 0.6) (layer B.Cu) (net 2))
 (segment (start 91.48 41.7) (end 90.24 40.46) (width 0.6) (layer B.Cu) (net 2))
 (segment (start 110.24 40.46) (end 109 41.7) (width 0.6) (layer B.Cu) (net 2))
 (segment (start 109 41.7) (end 91.48 41.7) (width 0.6) (layer B.Cu) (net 2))
 (segment (start 68.799999 37.799999) (end 72.799999 37.799999) (width 0.6) (layer B.Cu) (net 4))
 (segment (start 68 37) (end 68.799999 37.799999) (width 0.6) (layer B.Cu) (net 4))
 (segment (start 72.799999 37.799999) (end 74.2 39.2) (width 0.6) (layer B.Cu) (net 4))
 (segment (start 74.2 39.2) (end 87.6 39.2) (width 0.6) (layer B.Cu) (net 4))
 (segment (start 87.6 38.02) (end 87.6 39.2) (width 0.6) (layer B.Cu) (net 4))
 (segment (start 90.24 35.38) (end 87.6 38.02) (width 0.6) (layer B.Cu) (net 4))
 (segment (start 90.839999 35.979999) (end 90.979999 35.979999) (width 0.6) (layer B.Cu) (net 4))
 (segment (start 90.24 35.38) (end 90.839999 35.979999) (width 0.6) (layer B.Cu) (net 4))
 (segment (start 90.979999 35.979999) (end 94.2 39.2) (width 0.6) (layer B.Cu) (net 4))
 (segment (start 106.42 39.2) (end 110.24 35.38) (width 0.6) (layer B.Cu) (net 4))
 (segment (start 94.2 39.2) (end 106.42 39.2) (width 0.6) (layer B.Cu) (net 4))
 (segment (start 68.799999 34.799999) (end 72.399999 34.799999) (width 0.6) (layer B.Cu) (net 5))
 (segment (start 68 34) (end 68.799999 34.799999) (width 0.6) (layer B.Cu) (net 5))
 (segment (start 72.399999 34.799999) (end 74.3 36.7) (width 0.6) (layer B.Cu) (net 5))
 (segment (start 86.38 36.7) (end 90.24 32.84) (width 0.6) (layer B.Cu) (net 5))
 (segment (start 74.3 36.7) (end 86.38 36.7) (width 0.6) (layer B.Cu) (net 5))
 (segment (start 110.24 32.84) (end 105.78 37.3) (width 0.6) (layer B.Cu) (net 5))
 (segment (start 105.78 37.3) (end 96.4 37.3) (width 0.6) (layer B.Cu) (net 5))
 (segment (start 96.4 37.3) (end 95.7 36.6) (width 0.6) (layer B.Cu) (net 5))
 (segment (start 94 36.6) (end 90.24 32.84) (width 0.6) (layer B.Cu) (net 5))
 (segment (start 95.7 36.6) (end 94 36.6) (width 0.6) (layer B.Cu) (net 5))
 (segment (start 108.94 31.6) (end 110.24 30.3) (width 0.6) (layer B.Cu) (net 6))
 (segment (start 94.2 31.6) (end 108.94 31.6) (width 0.6) (layer B.Cu) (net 6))
 (segment (start 90.24 30.3) (end 92.9 30.3) (width 0.6) (layer B.Cu) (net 6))
 (segment (start 92.9 30.3) (end 94.2 31.6) (width 0.6) (layer B.Cu) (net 6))
 (segment (start 71.6 31.6) (end 68 28) (width 0.6) (layer B.Cu) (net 6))
 (segment (start 83.3 31.6) (end 71.6 31.6) (width 0.6) (layer B.Cu) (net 6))
 (segment (start 90.24 30.3) (end 84.6 30.3) (width 0.6) (layer B.Cu) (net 6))
 (segment (start 84.6 30.3) (end 83.3 31.6) (width 0.6) (layer B.Cu) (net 6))
 (segment (start 69.84 32.84) (end 75 32.84) (width 0.6) (layer B.Cu) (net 14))
 (segment (start 68 31) (end 69.84 32.84) (width 0.6) (layer B.Cu) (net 14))
 (segment (start 76.56 34.4) (end 75 32.84) (width 0.6) (layer B.Cu) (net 14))
 (segment (start 86.2 34.4) (end 76.56 34.4) (width 0.6) (layer B.Cu) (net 14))
 (segment (start 89 31.6) (end 86.2 34.4) (width 0.6) (layer B.Cu) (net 14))
 (segment (start 95 32.84) (end 92.24 32.84) (width 0.6) (layer B.Cu) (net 14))
 (segment (start 91 31.6) (end 89 31.6) (width 0.6) (layer B.Cu) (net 14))
 (segment (start 92.24 32.84) (end 91 31.6) (width 0.6) (layer B.Cu) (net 14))
 (segment (start 72.24 25) (end 75 27.76) (width 0.6) (layer B.Cu) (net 16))
 (segment (start 68 25) (end 72.24 25) (width 0.6) (layer B.Cu) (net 16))
 (segment (start 75.599999 27.160001) (end 75.599999 27.100001) (width 0.6) (layer B.Cu) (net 16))
 (segment (start 75 27.76) (end 75.599999 27.160001) (width 0.6) (layer B.Cu) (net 16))
 (segment (start 75.599999 27.100001) (end 78.8 23.9) (width 0.6) (layer B.Cu) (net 16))
 (segment (start 91.14 23.9) (end 95 27.76) (width 0.6) (layer B.Cu) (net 16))
 (segment (start 78.8 23.9) (end 91.14 23.9) (width 0.6) (layer B.Cu) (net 16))
 (segment (start 71.78 22) (end 75 25.22) (width 0.6) (layer B.Cu) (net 17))
 (segment (start 68 22) (end 71.78 22) (width 0.6) (layer B.Cu) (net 17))
 (segment (start 75 25.22) (end 79.12 21.1) (width 0.6) (layer B.Cu) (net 17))
 (segment (start 90.88 21.1) (end 95 25.22) (width 0.6) (layer B.Cu) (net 17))
 (segment (start 79.12 21.1) (end 90.88 21.1) (width 0.6) (layer B.Cu) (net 17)))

